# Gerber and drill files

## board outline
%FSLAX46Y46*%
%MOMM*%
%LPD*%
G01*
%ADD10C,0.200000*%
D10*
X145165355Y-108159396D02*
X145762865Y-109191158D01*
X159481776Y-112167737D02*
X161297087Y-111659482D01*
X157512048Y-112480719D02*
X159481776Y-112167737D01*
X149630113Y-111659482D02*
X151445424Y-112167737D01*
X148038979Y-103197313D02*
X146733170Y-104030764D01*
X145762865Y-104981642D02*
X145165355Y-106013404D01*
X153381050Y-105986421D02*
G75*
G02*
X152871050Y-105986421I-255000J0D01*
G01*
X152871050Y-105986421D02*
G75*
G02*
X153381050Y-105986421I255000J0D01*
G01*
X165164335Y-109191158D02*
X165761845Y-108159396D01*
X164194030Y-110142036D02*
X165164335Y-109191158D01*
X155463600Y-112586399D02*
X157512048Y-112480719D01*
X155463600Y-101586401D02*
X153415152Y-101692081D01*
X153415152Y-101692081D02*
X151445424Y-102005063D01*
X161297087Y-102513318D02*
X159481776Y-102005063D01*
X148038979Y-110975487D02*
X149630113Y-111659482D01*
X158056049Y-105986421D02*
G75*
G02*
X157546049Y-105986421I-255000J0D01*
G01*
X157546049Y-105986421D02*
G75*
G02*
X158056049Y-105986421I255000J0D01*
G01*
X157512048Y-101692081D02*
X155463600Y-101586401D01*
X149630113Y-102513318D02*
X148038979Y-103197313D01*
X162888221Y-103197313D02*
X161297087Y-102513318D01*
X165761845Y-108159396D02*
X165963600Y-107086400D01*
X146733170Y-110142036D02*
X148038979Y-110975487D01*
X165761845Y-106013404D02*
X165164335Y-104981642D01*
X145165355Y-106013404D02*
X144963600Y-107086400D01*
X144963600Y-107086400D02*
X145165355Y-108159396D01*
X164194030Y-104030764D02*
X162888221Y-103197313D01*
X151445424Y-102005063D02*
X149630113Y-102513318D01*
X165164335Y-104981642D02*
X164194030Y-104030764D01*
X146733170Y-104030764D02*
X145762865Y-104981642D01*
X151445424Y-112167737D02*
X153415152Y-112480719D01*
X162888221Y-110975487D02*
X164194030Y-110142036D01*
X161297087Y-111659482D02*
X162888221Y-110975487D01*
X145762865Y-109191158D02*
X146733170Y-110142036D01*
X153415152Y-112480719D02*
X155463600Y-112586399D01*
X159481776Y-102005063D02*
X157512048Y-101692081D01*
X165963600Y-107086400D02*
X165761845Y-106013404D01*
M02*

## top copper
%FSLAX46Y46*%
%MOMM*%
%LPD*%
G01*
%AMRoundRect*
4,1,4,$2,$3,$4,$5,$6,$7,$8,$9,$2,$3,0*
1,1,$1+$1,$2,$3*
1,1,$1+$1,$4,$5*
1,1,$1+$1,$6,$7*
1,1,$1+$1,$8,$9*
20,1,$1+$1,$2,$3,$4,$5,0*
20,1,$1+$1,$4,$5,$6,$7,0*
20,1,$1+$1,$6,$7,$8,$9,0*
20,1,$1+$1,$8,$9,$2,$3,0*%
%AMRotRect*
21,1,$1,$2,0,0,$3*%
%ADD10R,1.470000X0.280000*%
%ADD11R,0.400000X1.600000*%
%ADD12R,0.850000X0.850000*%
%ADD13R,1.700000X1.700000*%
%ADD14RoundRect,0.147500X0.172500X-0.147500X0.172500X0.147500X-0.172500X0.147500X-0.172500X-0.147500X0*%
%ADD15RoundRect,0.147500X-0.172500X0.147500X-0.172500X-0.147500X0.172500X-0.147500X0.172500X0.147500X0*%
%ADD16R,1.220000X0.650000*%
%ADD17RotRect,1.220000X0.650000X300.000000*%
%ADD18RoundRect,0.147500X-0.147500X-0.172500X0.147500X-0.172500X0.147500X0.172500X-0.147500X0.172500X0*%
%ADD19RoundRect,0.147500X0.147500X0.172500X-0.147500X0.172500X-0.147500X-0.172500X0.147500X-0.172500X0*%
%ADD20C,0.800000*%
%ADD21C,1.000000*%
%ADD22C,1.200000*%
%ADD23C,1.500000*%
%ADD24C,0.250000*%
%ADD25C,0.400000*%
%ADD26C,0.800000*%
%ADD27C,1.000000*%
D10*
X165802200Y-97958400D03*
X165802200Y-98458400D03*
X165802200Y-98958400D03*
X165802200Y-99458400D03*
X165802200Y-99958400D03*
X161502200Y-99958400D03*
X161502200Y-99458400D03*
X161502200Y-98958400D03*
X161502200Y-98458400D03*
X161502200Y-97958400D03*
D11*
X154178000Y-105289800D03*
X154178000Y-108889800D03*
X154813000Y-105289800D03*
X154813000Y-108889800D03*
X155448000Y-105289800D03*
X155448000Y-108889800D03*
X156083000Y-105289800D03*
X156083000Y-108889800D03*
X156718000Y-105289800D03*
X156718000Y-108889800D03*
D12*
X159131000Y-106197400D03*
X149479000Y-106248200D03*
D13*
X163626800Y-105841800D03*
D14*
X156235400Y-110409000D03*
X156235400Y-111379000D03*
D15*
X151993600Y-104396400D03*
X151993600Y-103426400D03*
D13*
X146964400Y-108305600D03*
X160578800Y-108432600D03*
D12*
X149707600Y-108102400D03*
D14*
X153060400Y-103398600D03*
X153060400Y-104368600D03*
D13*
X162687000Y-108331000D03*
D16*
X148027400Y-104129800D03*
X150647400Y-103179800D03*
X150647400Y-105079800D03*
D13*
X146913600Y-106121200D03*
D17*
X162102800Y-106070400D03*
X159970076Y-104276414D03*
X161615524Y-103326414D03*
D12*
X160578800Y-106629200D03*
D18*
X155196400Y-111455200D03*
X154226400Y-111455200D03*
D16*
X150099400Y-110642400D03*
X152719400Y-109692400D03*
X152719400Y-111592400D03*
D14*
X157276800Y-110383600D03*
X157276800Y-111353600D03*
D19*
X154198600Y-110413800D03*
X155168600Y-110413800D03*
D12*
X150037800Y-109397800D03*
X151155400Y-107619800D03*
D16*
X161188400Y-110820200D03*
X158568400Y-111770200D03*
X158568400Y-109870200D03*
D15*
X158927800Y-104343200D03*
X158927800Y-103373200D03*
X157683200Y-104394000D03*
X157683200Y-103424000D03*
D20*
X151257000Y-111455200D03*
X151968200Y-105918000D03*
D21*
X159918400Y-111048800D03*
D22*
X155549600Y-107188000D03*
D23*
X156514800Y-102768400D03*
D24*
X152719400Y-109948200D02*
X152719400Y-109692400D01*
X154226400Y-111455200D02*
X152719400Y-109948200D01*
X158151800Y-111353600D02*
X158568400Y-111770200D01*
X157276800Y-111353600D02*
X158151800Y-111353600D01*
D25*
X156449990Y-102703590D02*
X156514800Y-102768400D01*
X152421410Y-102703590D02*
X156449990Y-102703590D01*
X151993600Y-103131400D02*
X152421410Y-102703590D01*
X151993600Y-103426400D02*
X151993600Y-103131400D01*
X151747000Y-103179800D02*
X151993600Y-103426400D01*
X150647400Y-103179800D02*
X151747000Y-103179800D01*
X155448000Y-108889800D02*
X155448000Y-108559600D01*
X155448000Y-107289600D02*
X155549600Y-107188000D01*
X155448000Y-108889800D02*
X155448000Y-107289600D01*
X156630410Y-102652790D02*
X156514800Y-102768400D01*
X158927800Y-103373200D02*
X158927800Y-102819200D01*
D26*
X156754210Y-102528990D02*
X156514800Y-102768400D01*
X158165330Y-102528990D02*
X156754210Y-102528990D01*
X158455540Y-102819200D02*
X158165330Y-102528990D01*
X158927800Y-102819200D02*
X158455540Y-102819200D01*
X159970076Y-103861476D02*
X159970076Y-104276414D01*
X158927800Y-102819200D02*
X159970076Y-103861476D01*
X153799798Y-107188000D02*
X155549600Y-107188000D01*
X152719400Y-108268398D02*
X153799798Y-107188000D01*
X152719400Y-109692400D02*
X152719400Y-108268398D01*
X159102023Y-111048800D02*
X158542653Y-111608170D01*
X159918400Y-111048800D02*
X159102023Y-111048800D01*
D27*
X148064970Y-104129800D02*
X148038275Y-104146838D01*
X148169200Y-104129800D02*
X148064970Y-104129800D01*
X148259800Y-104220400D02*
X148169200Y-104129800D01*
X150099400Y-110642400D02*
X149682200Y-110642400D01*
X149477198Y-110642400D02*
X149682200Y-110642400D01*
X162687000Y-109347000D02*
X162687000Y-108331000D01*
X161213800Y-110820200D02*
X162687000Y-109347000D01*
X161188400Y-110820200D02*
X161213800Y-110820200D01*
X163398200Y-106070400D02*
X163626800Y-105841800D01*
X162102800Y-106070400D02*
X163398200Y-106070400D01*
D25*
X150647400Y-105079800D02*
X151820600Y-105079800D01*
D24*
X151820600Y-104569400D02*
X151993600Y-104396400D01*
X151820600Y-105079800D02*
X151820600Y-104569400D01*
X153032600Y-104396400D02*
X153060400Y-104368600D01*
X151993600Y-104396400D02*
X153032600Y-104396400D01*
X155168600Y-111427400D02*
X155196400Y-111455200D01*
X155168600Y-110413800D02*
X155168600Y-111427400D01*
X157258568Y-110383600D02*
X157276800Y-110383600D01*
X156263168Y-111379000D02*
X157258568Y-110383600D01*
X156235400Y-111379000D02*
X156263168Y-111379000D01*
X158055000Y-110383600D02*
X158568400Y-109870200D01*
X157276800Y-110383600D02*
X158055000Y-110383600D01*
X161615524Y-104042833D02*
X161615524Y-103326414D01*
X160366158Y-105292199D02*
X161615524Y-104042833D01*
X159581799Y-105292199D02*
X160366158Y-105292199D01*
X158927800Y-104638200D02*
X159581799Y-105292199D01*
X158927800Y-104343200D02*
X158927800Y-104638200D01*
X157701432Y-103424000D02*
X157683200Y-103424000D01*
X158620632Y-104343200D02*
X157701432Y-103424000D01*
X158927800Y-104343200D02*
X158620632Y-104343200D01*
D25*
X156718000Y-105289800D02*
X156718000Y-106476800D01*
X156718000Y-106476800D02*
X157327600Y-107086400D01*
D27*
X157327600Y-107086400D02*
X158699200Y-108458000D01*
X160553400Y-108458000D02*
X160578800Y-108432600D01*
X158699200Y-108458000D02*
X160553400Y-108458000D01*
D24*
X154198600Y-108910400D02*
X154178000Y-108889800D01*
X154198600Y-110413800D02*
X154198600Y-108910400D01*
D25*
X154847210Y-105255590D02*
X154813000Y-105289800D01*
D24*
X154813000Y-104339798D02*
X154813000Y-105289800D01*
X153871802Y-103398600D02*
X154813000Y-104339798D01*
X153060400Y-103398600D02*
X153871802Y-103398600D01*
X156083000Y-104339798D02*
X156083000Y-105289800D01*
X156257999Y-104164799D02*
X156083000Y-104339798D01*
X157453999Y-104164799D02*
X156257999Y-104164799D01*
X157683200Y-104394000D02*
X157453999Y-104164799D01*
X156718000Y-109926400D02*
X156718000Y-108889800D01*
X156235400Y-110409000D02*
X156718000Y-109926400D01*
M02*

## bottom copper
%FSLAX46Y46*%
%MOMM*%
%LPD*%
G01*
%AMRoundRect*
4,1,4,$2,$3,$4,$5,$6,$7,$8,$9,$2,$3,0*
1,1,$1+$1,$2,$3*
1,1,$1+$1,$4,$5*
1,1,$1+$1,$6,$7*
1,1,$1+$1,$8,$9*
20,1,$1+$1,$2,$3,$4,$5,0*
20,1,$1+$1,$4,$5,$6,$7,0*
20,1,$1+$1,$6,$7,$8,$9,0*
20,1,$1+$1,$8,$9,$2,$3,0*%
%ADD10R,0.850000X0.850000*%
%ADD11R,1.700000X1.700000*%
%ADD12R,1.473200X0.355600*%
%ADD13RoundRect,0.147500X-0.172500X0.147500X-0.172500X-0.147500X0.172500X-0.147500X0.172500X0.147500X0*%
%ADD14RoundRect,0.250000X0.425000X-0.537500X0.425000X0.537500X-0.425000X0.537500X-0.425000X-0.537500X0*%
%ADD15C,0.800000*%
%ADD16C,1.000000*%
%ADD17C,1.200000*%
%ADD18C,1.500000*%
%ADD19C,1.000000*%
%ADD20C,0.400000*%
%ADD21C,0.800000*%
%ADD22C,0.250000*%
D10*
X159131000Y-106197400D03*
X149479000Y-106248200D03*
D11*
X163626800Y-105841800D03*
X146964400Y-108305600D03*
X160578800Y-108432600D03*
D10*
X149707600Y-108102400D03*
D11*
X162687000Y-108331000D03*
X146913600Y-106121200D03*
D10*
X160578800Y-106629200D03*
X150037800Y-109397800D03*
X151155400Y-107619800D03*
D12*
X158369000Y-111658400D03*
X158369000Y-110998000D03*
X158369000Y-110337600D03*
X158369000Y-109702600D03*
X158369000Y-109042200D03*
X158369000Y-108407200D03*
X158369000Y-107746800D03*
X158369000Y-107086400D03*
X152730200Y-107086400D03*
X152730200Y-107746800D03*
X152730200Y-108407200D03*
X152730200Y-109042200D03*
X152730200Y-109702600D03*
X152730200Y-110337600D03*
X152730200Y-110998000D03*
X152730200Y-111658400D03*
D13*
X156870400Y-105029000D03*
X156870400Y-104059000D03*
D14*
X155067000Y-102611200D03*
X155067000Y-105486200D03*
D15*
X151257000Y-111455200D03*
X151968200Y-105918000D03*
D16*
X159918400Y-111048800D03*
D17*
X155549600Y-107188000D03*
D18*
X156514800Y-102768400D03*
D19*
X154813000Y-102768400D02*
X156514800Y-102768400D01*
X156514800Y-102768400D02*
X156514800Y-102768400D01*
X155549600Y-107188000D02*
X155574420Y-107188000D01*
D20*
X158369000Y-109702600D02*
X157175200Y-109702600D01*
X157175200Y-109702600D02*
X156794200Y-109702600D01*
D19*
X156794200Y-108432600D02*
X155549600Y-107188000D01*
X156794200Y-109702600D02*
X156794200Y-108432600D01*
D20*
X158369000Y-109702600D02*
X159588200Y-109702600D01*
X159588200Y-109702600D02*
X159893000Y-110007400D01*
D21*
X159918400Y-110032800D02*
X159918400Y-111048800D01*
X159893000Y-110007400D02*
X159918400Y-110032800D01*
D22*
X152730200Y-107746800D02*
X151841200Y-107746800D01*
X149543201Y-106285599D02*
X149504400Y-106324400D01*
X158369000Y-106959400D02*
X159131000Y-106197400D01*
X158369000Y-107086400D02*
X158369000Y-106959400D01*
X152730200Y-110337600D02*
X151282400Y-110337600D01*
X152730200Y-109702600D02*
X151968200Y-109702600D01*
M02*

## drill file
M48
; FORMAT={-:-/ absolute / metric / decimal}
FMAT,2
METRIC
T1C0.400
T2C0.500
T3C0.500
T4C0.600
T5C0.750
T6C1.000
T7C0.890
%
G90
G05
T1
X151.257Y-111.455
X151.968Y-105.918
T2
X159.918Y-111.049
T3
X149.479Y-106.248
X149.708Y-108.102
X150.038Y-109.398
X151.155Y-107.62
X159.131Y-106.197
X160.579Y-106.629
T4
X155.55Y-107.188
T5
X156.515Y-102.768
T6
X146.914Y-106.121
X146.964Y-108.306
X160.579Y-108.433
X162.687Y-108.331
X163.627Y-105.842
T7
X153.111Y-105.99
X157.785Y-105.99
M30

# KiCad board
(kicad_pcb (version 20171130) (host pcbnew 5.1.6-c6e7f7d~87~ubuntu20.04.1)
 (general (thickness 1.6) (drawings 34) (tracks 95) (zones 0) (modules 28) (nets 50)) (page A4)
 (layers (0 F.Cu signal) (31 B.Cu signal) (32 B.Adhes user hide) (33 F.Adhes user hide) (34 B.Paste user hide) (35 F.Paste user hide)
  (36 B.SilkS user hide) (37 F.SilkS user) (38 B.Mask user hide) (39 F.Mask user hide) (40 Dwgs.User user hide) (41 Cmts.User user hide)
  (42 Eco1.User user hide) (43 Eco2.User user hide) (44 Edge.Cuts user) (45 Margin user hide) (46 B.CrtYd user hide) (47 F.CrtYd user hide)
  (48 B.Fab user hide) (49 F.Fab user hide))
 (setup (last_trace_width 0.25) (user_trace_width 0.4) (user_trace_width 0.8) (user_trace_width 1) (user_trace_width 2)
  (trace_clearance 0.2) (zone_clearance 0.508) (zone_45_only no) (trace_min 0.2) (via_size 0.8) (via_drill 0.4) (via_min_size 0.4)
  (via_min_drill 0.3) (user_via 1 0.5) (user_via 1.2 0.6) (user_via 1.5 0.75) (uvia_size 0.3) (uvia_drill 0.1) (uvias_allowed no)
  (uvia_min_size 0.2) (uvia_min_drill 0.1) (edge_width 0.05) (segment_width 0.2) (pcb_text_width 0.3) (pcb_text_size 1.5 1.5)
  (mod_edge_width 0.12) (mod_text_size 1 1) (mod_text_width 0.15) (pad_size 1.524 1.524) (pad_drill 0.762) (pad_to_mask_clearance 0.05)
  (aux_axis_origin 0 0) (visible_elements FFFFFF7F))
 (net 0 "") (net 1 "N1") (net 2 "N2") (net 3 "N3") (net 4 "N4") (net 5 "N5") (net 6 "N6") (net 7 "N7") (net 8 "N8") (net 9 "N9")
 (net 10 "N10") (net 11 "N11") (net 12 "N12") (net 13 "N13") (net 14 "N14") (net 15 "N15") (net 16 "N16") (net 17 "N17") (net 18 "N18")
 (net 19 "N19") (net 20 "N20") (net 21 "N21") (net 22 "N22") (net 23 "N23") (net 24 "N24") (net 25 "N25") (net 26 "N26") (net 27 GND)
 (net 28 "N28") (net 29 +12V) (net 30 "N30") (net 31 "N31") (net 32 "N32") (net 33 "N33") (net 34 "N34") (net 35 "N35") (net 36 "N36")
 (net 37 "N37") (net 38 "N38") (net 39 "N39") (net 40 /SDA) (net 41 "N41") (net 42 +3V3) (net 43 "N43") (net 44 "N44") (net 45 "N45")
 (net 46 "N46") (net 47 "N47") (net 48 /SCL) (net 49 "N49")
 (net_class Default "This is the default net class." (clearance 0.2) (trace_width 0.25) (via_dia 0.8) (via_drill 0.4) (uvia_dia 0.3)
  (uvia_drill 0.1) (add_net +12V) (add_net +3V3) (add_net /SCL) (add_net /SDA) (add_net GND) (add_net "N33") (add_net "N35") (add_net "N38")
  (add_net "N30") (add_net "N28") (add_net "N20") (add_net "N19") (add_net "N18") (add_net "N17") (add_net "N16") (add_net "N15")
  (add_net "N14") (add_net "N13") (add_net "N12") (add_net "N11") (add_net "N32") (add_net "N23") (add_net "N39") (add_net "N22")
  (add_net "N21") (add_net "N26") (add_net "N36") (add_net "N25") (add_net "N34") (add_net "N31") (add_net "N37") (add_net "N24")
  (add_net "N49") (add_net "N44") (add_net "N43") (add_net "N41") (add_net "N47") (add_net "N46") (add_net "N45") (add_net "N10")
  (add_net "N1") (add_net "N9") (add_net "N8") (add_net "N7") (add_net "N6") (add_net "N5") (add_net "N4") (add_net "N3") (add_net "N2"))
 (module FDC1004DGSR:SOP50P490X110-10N (layer F.Cu) (at 163.6522 98.9584)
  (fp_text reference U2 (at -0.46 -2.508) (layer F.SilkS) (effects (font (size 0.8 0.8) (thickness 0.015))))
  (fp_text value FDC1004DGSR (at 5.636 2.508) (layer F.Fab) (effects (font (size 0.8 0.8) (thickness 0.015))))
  (pad 10 smd rect (at 2.15 -1) (size 1.47 0.28) (layers F.Cu F.Paste F.Mask) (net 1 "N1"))
  (pad 9 smd rect (at 2.15 -0.5) (size 1.47 0.28) (layers F.Cu F.Paste F.Mask) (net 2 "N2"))
  (pad 8 smd rect (at 2.15 0) (size 1.47 0.28) (layers F.Cu F.Paste F.Mask) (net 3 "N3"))
  (pad 7 smd rect (at 2.15 0.5) (size 1.47 0.28) (layers F.Cu F.Paste F.Mask) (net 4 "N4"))
  (pad 6 smd rect (at 2.15 1) (size 1.47 0.28) (layers F.Cu F.Paste F.Mask) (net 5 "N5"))
  (pad 5 smd rect (at -2.15 1) (size 1.47 0.28) (layers F.Cu F.Paste F.Mask) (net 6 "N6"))
  (pad 4 smd rect (at -2.15 0.5) (size 1.47 0.28) (layers F.Cu F.Paste F.Mask) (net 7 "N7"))
  (pad 3 smd rect (at -2.15 0) (size 1.47 0.28) (layers F.Cu F.Paste F.Mask) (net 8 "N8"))
  (pad 2 smd rect (at -2.15 -0.5) (size 1.47 0.28) (layers F.Cu F.Paste F.Mask) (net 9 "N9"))
  (pad 1 smd rect (at -2.15 -1) (size 1.47 0.28) (layers F.Cu F.Paste F.Mask) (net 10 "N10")))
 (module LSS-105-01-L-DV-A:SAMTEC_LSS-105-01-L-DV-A (layer F.Cu) (at 156.718 108.8898)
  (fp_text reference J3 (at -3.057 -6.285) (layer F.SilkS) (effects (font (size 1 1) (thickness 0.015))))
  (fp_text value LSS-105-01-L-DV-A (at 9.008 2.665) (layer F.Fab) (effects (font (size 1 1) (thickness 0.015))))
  (pad 10 smd rect (at -2.54 -3.6) (size 0.4 1.6) (layers F.Cu F.Paste F.Mask) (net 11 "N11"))
  (pad 09 smd rect (at -2.54 0) (size 0.4 1.6) (layers F.Cu F.Paste F.Mask) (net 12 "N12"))
  (pad 08 smd rect (at -1.905 -3.6) (size 0.4 1.6) (layers F.Cu F.Paste F.Mask) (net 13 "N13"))
  (pad 07 smd rect (at -1.905 0) (size 0.4 1.6) (layers F.Cu F.Paste F.Mask) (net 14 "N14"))
  (pad 06 smd rect (at -1.27 -3.6) (size 0.4 1.6) (layers F.Cu F.Paste F.Mask) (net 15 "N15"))
  (pad 05 smd rect (at -1.27 0) (size 0.4 1.6) (layers F.Cu F.Paste F.Mask) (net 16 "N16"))
  (pad 04 smd rect (at -0.635 -3.6) (size 0.4 1.6) (layers F.Cu F.Paste F.Mask) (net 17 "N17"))
  (pad 03 smd rect (at -0.635 0) (size 0.4 1.6) (layers F.Cu F.Paste F.Mask) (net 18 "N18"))
  (pad 02 smd rect (at 0 -3.6) (size 0.4 1.6) (layers F.Cu F.Paste F.Mask) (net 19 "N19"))
  (pad 01 smd rect (at 0 0) (size 0.4 1.6) (layers F.Cu F.Paste F.Mask) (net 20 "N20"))
  (pad None np_thru_hole circle (at 1.067 -2.9) (size 0.89 0.89) (drill 0.89) (layers *.Cu *.Mask))
  (pad None np_thru_hole circle (at -3.607 -2.9) (size 0.89 0.89) (drill 0.89) (layers *.Cu *.Mask)))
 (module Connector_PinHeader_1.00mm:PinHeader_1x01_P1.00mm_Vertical (layer F.Cu) (at 159.131 106.1974)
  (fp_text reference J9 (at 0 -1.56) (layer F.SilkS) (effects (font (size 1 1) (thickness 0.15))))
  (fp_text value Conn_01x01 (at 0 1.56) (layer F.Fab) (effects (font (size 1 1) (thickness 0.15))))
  (pad 1 thru_hole rect (at 0 0) (size 0.85 0.85) (drill 0.5) (layers *.Cu *.Mask) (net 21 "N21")))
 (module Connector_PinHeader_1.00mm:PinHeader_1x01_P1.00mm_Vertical (layer F.Cu) (at 149.479 106.2482)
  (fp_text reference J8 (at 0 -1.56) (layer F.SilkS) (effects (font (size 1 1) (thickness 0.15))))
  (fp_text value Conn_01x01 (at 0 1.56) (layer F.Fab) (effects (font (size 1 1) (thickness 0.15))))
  (pad 1 thru_hole rect (at 0 0) (size 0.85 0.85) (drill 0.5) (layers *.Cu *.Mask) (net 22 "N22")))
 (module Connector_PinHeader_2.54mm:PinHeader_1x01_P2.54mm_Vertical (layer F.Cu) (at 163.6268 105.8418)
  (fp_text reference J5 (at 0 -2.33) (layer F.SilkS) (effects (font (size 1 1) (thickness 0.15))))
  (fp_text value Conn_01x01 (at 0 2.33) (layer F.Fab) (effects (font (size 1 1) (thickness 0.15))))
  (pad 1 thru_hole rect (at 0 0) (size 1.7 1.7) (drill 1) (layers *.Cu *.Mask) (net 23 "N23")))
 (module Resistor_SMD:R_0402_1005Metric (layer F.Cu) (at 156.2354 110.894 90)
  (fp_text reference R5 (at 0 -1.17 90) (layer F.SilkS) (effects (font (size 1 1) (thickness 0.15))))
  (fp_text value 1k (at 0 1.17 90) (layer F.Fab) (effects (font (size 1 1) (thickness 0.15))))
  (pad 2 smd roundrect (at 0.485 0 90) (size 0.59 0.64) (layers F.Cu F.Paste F.Mask) (roundrect_rratio 0.25) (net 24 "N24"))
  (pad 1 smd roundrect (at -0.485 0 90) (size 0.59 0.64) (layers F.Cu F.Paste F.Mask) (roundrect_rratio 0.25) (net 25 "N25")))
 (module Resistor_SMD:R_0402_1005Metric (layer F.Cu) (at 151.9936 103.9114 270)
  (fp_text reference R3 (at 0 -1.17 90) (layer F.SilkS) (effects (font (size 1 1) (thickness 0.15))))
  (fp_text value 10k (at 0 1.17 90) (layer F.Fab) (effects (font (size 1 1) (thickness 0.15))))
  (pad 2 smd roundrect (at 0.485 0 270) (size 0.59 0.64) (layers F.Cu F.Paste F.Mask) (roundrect_rratio 0.25) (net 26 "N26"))
  (pad 1 smd roundrect (at -0.485 0 270) (size 0.59 0.64) (layers F.Cu F.Paste F.Mask) (roundrect_rratio 0.25) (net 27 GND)))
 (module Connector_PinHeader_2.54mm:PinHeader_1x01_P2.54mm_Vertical (layer F.Cu) (at 146.9644 108.3056)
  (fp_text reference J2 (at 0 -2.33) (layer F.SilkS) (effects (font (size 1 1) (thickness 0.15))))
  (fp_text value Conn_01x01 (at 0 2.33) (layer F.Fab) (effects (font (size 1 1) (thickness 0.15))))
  (pad 1 thru_hole rect (at 0 0) (size 1.7 1.7) (drill 1) (layers *.Cu *.Mask) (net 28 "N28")))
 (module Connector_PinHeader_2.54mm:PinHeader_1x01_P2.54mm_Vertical (layer F.Cu) (at 160.5788 108.4326)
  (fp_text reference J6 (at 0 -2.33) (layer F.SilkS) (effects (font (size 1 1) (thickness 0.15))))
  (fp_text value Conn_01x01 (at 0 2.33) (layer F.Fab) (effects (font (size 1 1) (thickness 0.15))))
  (pad 1 thru_hole rect (at 0 0) (size 1.7 1.7) (drill 1) (layers *.Cu *.Mask) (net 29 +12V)))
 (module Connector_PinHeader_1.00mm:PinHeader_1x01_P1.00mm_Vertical (layer F.Cu) (at 149.7076 108.1024)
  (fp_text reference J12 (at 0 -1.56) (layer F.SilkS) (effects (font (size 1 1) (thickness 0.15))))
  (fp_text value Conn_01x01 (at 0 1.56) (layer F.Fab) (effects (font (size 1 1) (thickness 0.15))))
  (pad 1 thru_hole rect (at 0 0) (size 0.85 0.85) (drill 0.5) (layers *.Cu *.Mask) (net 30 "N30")))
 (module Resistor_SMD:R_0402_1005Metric (layer F.Cu) (at 153.0604 103.8836 90)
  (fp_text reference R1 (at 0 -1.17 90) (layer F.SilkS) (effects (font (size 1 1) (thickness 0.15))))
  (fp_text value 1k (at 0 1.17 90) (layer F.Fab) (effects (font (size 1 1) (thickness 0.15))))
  (pad 2 smd roundrect (at 0.485 0 90) (size 0.59 0.64) (layers F.Cu F.Paste F.Mask) (roundrect_rratio 0.25) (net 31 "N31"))
  (pad 1 smd roundrect (at -0.485 0 90) (size 0.59 0.64) (layers F.Cu F.Paste F.Mask) (roundrect_rratio 0.25) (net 26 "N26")))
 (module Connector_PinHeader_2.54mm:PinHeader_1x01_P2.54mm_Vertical (layer F.Cu) (at 162.687 108.331)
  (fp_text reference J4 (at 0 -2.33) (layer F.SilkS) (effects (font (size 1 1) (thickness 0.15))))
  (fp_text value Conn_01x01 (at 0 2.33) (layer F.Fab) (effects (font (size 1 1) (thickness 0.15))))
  (pad 1 thru_hole rect (at 0 0) (size 1.7 1.7) (drill 1) (layers *.Cu *.Mask) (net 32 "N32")))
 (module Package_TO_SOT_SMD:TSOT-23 (layer F.Cu) (at 149.3374 104.1298 180)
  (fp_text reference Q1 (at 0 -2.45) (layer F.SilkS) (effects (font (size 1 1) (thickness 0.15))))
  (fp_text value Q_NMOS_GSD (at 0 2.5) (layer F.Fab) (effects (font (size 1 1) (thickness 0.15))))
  (pad 3 smd rect (at 1.31 0 180) (size 1.22 0.65) (layers F.Cu F.Paste F.Mask) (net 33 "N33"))
  (pad 2 smd rect (at -1.31 0.95 180) (size 1.22 0.65) (layers F.Cu F.Paste F.Mask) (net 27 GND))
  (pad 1 smd rect (at -1.31 -0.95 180) (size 1.22 0.65) (layers F.Cu F.Paste F.Mask) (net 26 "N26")))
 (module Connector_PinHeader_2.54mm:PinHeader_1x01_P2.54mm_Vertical (layer F.Cu) (at 146.9136 106.1212)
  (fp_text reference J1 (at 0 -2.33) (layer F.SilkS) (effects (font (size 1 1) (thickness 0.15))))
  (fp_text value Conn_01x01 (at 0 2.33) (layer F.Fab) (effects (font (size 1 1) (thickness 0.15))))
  (pad 1 thru_hole rect (at 0 0) (size 1.7 1.7) (drill 1) (layers *.Cu *.Mask) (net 33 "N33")))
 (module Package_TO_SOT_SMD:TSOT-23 (layer F.Cu) (at 161.4478 104.935907 300)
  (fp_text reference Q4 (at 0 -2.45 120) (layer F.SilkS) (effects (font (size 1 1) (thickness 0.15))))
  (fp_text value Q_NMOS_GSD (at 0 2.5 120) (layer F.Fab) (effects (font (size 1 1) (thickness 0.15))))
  (pad 3 smd rect (at 1.31 0 300) (size 1.22 0.65) (layers F.Cu F.Paste F.Mask) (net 23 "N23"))
  (pad 2 smd rect (at -1.31 0.95 300) (size 1.22 0.65) (layers F.Cu F.Paste F.Mask) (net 27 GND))
  (pad 1 smd rect (at -1.31 -0.95 300) (size 1.22 0.65) (layers F.Cu F.Paste F.Mask) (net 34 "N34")))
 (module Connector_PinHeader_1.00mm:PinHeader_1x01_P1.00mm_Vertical (layer F.Cu) (at 160.5788 106.6292)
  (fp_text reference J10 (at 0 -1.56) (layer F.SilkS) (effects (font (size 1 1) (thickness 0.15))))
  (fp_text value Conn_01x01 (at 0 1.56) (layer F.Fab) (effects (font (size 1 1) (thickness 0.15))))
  (pad 1 thru_hole rect (at 0 0) (size 0.85 0.85) (drill 0.5) (layers *.Cu *.Mask) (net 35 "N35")))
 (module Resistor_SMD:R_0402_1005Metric (layer F.Cu) (at 154.7114 111.4552)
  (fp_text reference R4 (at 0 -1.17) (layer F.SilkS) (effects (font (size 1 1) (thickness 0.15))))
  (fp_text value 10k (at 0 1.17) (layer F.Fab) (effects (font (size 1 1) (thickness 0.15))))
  (pad 2 smd roundrect (at 0.485 0) (size 0.59 0.64) (layers F.Cu F.Paste F.Mask) (roundrect_rratio 0.25) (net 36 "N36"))
  (pad 1 smd roundrect (at -0.485 0) (size 0.59 0.64) (layers F.Cu F.Paste F.Mask) (roundrect_rratio 0.25) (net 27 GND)))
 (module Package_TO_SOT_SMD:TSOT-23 (layer F.Cu) (at 151.4094 110.6424 180)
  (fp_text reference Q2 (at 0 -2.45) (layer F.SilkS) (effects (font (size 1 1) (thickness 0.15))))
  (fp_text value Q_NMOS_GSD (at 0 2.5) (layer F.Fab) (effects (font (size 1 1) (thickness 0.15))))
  (pad 3 smd rect (at 1.31 0 180) (size 1.22 0.65) (layers F.Cu F.Paste F.Mask) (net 28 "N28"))
  (pad 2 smd rect (at -1.31 0.95 180) (size 1.22 0.65) (layers F.Cu F.Paste F.Mask) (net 27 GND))
  (pad 1 smd rect (at -1.31 -0.95 180) (size 1.22 0.65) (layers F.Cu F.Paste F.Mask) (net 36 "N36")))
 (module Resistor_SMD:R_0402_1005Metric (layer F.Cu) (at 157.2768 110.8686 90)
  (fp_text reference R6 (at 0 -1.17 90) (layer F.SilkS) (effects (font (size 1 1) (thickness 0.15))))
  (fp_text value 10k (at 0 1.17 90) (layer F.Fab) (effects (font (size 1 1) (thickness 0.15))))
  (pad 2 smd roundrect (at 0.485 0 90) (size 0.59 0.64) (layers F.Cu F.Paste F.Mask) (roundrect_rratio 0.25) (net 25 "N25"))
  (pad 1 smd roundrect (at -0.485 0 90) (size 0.59 0.64) (layers F.Cu F.Paste F.Mask) (roundrect_rratio 0.25) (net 27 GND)))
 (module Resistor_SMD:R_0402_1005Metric (layer F.Cu) (at 154.6836 110.4138 180)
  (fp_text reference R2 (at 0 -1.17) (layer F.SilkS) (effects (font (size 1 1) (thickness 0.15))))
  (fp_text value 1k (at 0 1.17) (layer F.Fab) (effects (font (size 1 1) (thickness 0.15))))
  (pad 2 smd roundrect (at 0.485 0 180) (size 0.59 0.64) (layers F.Cu F.Paste F.Mask) (roundrect_rratio 0.25) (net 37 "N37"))
  (pad 1 smd roundrect (at -0.485 0 180) (size 0.59 0.64) (layers F.Cu F.Paste F.Mask) (roundrect_rratio 0.25) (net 36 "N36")))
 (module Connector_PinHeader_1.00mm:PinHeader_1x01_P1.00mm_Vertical (layer F.Cu) (at 150.0378 109.3978)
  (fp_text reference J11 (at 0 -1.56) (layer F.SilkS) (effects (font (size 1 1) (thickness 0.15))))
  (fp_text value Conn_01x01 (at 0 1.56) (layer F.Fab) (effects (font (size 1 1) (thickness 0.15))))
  (pad 1 thru_hole rect (at 0 0) (size 0.85 0.85) (drill 0.5) (layers *.Cu *.Mask) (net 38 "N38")))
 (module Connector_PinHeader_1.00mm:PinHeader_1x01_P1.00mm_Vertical (layer F.Cu) (at 151.1554 107.6198)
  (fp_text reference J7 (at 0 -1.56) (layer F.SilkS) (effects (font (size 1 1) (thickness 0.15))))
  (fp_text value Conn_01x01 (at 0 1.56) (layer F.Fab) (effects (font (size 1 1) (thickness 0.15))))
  (pad 1 thru_hole rect (at 0 0) (size 0.85 0.85) (drill 0.5) (layers *.Cu *.Mask) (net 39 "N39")))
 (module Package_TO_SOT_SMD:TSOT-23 (layer F.Cu) (at 159.8784 110.8202)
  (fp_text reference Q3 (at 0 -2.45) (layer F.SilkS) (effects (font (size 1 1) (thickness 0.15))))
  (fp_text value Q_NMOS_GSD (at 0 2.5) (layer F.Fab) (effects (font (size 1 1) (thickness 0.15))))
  (pad 3 smd rect (at 1.31 0) (size 1.22 0.65) (layers F.Cu F.Paste F.Mask) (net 32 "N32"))
  (pad 2 smd rect (at -1.31 0.95) (size 1.22 0.65) (layers F.Cu F.Paste F.Mask) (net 27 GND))
  (pad 1 smd rect (at -1.31 -0.95) (size 1.22 0.65) (layers F.Cu F.Paste F.Mask) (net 25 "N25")))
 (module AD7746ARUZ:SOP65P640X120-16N (layer B.Cu) (at 155.5496 109.3724)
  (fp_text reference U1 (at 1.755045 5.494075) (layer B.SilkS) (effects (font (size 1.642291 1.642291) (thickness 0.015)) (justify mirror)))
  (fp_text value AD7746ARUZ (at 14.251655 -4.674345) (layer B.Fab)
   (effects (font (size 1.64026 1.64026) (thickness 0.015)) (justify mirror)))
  (pad 16 smd rect (at 2.8194 2.286) (size 1.4732 0.3556) (layers B.Cu B.Paste B.Mask) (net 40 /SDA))
  (pad 15 smd rect (at 2.8194 1.6256) (size 1.4732 0.3556) (layers B.Cu B.Paste B.Mask) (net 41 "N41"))
  (pad 14 smd rect (at 2.8194 0.9652) (size 1.4732 0.3556) (layers B.Cu B.Paste B.Mask) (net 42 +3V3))
  (pad 13 smd rect (at 2.8194 0.3302) (size 1.4732 0.3556) (layers B.Cu B.Paste B.Mask) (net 27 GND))
  (pad 12 smd rect (at 2.8194 -0.3302) (size 1.4732 0.3556) (layers B.Cu B.Paste B.Mask) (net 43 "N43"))
  (pad 11 smd rect (at 2.8194 -0.9652) (size 1.4732 0.3556) (layers B.Cu B.Paste B.Mask) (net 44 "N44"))
  (pad 10 smd rect (at 2.8194 -1.6256) (size 1.4732 0.3556) (layers B.Cu B.Paste B.Mask) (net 35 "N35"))
  (pad 9 smd rect (at 2.8194 -2.286) (size 1.4732 0.3556) (layers B.Cu B.Paste B.Mask) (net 21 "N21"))
  (pad 8 smd rect (at -2.8194 -2.286) (size 1.4732 0.3556) (layers B.Cu B.Paste B.Mask) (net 22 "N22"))
  (pad 7 smd rect (at -2.8194 -1.6256) (size 1.4732 0.3556) (layers B.Cu B.Paste B.Mask) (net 39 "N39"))
  (pad 6 smd rect (at -2.8194 -0.9652) (size 1.4732 0.3556) (layers B.Cu B.Paste B.Mask) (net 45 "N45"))
  (pad 5 smd rect (at -2.8194 -0.3302) (size 1.4732 0.3556) (layers B.Cu B.Paste B.Mask) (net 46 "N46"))
  (pad 4 smd rect (at -2.8194 0.3302) (size 1.4732 0.3556) (layers B.Cu B.Paste B.Mask) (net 30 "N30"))
  (pad 3 smd rect (at -2.8194 0.9652) (size 1.4732 0.3556) (layers B.Cu B.Paste B.Mask) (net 38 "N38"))
  (pad 2 smd rect (at -2.8194 1.6256) (size 1.4732 0.3556) (layers B.Cu B.Paste B.Mask) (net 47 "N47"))
  (pad 1 smd rect (at -2.8194 2.286) (size 1.4732 0.3556) (layers B.Cu B.Paste B.Mask) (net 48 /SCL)))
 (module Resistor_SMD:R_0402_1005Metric (layer F.Cu) (at 158.9278 103.8582 270)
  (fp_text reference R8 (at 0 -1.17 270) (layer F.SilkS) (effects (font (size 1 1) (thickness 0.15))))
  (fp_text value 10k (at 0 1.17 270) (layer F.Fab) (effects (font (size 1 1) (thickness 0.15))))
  (pad 2 smd roundrect (at 0.485 0 270) (size 0.59 0.64) (layers F.Cu F.Paste F.Mask) (roundrect_rratio 0.25) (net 34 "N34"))
  (pad 1 smd roundrect (at -0.485 0 270) (size 0.59 0.64) (layers F.Cu F.Paste F.Mask) (roundrect_rratio 0.25) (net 27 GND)))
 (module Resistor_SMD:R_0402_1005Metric (layer F.Cu) (at 157.6832 103.909 270)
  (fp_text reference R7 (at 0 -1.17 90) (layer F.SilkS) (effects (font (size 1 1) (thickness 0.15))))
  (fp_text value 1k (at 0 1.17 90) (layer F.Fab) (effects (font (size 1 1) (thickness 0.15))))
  (pad 2 smd roundrect (at 0.485 0 270) (size 0.59 0.64) (layers F.Cu F.Paste F.Mask) (roundrect_rratio 0.25) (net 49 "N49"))
  (pad 1 smd roundrect (at -0.485 0 270) (size 0.59 0.64) (layers F.Cu F.Paste F.Mask) (roundrect_rratio 0.25) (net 34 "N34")))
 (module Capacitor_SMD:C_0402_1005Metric (layer B.Cu) (at 156.8704 104.544 270)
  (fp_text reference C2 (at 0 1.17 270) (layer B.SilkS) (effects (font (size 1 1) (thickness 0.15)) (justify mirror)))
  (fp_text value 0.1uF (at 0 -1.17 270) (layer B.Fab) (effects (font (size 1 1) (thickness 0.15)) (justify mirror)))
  (pad 2 smd roundrect (at 0.485 0 270) (size 0.59 0.64) (layers B.Cu B.Paste B.Mask) (roundrect_rratio 0.25) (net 27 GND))
  (pad 1 smd roundrect (at -0.485 0 270) (size 0.59 0.64) (layers B.Cu B.Paste B.Mask) (roundrect_rratio 0.25) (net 42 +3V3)))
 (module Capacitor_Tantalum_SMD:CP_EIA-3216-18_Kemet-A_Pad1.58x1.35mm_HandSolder (layer B.Cu) (at 155.067 104.0487 90)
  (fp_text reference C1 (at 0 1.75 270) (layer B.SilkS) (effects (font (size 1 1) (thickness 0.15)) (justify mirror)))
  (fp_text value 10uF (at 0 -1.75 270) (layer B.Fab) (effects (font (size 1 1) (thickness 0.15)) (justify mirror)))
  (pad 2 smd roundrect (at 1.4375 0 90) (size 1.575 1.35) (layers B.Cu B.Paste B.Mask) (roundrect_rratio 0.185185) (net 27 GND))
  (pad 1 smd roundrect (at -1.4375 0 90) (size 1.575 1.35) (layers B.Cu B.Paste B.Mask) (roundrect_rratio 0.185185) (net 42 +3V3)))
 (gr_line (start 145.165355 108.159396) (end 145.762865 109.191158) (layer Edge.Cuts) (width 0.2))
 (gr_line (start 159.481776 112.167737) (end 161.297087 111.659482) (layer Edge.Cuts) (width 0.2))
 (gr_line (start 157.512048 112.480719) (end 159.481776 112.167737) (layer Edge.Cuts) (width 0.2))
 (gr_line (start 149.630113 111.659482) (end 151.445424 112.167737) (layer Edge.Cuts) (width 0.2))
 (gr_line (start 148.038979 103.197313) (end 146.73317 104.030764) (layer Edge.Cuts) (width 0.2))
 (gr_line (start 145.762865 104.981642) (end 145.165355 106.013404) (layer Edge.Cuts) (width 0.2))
 (gr_circle (center 153.12605 105.986421) (end 153.38105 105.986421) (layer Edge.Cuts) (width 0.2))
 (gr_line (start 165.164335 109.191158) (end 165.761845 108.159396) (layer Edge.Cuts) (width 0.2))
 (gr_line (start 164.19403 110.142036) (end 165.164335 109.191158) (layer Edge.Cuts) (width 0.2))
 (gr_line (start 155.4636 112.586399) (end 157.512048 112.480719) (layer Edge.Cuts) (width 0.2))
 (gr_line (start 155.4636 101.586401) (end 153.415152 101.692081) (layer Edge.Cuts) (width 0.2))
 (gr_line (start 153.415152 101.692081) (end 151.445424 102.005063) (layer Edge.Cuts) (width 0.2))
 (gr_line (start 161.297087 102.513318) (end 159.481776 102.005063) (layer Edge.Cuts) (width 0.2))
 (gr_line (start 148.038979 110.975487) (end 149.630113 111.659482) (layer Edge.Cuts) (width 0.2))
 (gr_circle (center 157.801049 105.986421) (end 158.056049 105.986421) (layer Edge.Cuts) (width 0.2))
 (gr_line (start 157.512048 101.692081) (end 155.4636 101.586401) (layer Edge.Cuts) (width 0.2))
 (gr_line (start 149.630113 102.513318) (end 148.038979 103.197313) (layer Edge.Cuts) (width 0.2))
 (gr_line (start 162.888221 103.197313) (end 161.297087 102.513318) (layer Edge.Cuts) (width 0.2))
 (gr_line (start 165.761845 108.159396) (end 165.9636 107.0864) (layer Edge.Cuts) (width 0.2))
 (gr_line (start 146.73317 110.142036) (end 148.038979 110.975487) (layer Edge.Cuts) (width 0.2))
 (gr_line (start 165.761845 106.013404) (end 165.164335 104.981642) (layer Edge.Cuts) (width 0.2))
 (gr_line (start 145.165355 106.013404) (end 144.9636 107.0864) (layer Edge.Cuts) (width 0.2))
 (gr_line (start 144.9636 107.0864) (end 145.165355 108.159396) (layer Edge.Cuts) (width 0.2))
 (gr_line (start 164.19403 104.030764) (end 162.888221 103.197313) (layer Edge.Cuts) (width 0.2))
 (gr_line (start 151.445424 102.005063) (end 149.630113 102.513318) (layer Edge.Cuts) (width 0.2))
 (gr_line (start 165.164335 104.981642) (end 164.19403 104.030764) (layer Edge.Cuts) (width 0.2))
 (gr_line (start 146.73317 104.030764) (end 145.762865 104.981642) (layer Edge.Cuts) (width 0.2))
 (gr_line (start 151.445424 112.167737) (end 153.415152 112.480719) (layer Edge.Cuts) (width 0.2))
 (gr_line (start 162.888221 110.975487) (end 164.19403 110.142036) (layer Edge.Cuts) (width 0.2))
 (gr_line (start 161.297087 111.659482) (end 162.888221 110.975487) (layer Edge.Cuts) (width 0.2))
 (gr_line (start 145.762865 109.191158) (end 146.73317 110.142036) (layer Edge.Cuts) (width 0.2))
 (gr_line (start 153.415152 112.480719) (end 155.4636 112.586399) (layer Edge.Cuts) (width 0.2))
 (gr_line (start 159.481776 102.005063) (end 157.512048 101.692081) (layer Edge.Cuts) (width 0.2))
 (gr_line (start 165.9636 107.0864) (end 165.761845 106.013404) (layer Edge.Cuts) (width 0.2))
 (via (at 151.257 111.4552) (size 0.8) (drill 0.4) (layers F.Cu B.Cu) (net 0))
 (via (at 151.9682 105.918) (size 0.8) (drill 0.4) (layers F.Cu B.Cu) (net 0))
 (via (at 159.9184 111.0488) (size 1) (drill 0.5) (layers F.Cu B.Cu) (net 27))
 (via (at 155.5496 107.188) (size 1.2) (drill 0.6) (layers F.Cu B.Cu) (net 27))
 (segment (start 152.7194 109.9482) (end 152.7194 109.6924) (width 0.25) (layer F.Cu) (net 27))
 (segment (start 154.2264 111.4552) (end 152.7194 109.9482) (width 0.25) (layer F.Cu) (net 27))
 (segment (start 158.1518 111.3536) (end 158.5684 111.7702) (width 0.25) (layer F.Cu) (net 27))
 (segment (start 157.2768 111.3536) (end 158.1518 111.3536) (width 0.25) (layer F.Cu) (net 27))
 (segment (start 154.813 102.7684) (end 156.5148 102.7684) (width 1) (layer B.Cu) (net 27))
 (segment (start 156.5148 102.7684) (end 156.5148 102.7684) (width 1) (layer B.Cu) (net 27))
 (via (at 156.5148 102.7684) (size 1.5) (drill 0.75) (layers F.Cu B.Cu) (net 27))
 (segment (start 156.44999 102.70359) (end 156.5148 102.7684) (width 0.4) (layer F.Cu) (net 27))
 (segment (start 152.42141 102.70359) (end 156.44999 102.70359) (width 0.4) (layer F.Cu) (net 27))
 (segment (start 151.9936 103.1314) (end 152.42141 102.70359) (width 0.4) (layer F.Cu) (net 27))
 (segment (start 151.9936 103.4264) (end 151.9936 103.1314) (width 0.4) (layer F.Cu) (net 27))
 (segment (start 151.747 103.1798) (end 151.9936 103.4264) (width 0.4) (layer F.Cu) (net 27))
 (segment (start 150.6474 103.1798) (end 151.747 103.1798) (width 0.4) (layer F.Cu) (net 27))
 (segment (start 155.448 108.8898) (end 155.448 108.5596) (width 0.4) (layer F.Cu) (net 27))
 (segment (start 155.448 107.2896) (end 155.5496 107.188) (width 0.4) (layer F.Cu) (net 27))
 (segment (start 155.448 108.8898) (end 155.448 107.2896) (width 0.4) (layer F.Cu) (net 27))
 (segment (start 155.5496 107.188) (end 155.57442 107.188) (width 1) (layer B.Cu) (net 27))
 (segment (start 156.63041 102.65279) (end 156.5148 102.7684) (width 0.4) (layer F.Cu) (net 27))
 (segment (start 158.9278 103.3732) (end 158.9278 102.8192) (width 0.4) (layer F.Cu) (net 27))
 (segment (start 156.75421 102.52899) (end 156.5148 102.7684) (width 0.8) (layer F.Cu) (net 27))
 (segment (start 158.16533 102.52899) (end 156.75421 102.52899) (width 0.8) (layer F.Cu) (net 27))
 (segment (start 158.45554 102.8192) (end 158.16533 102.52899) (width 0.8) (layer F.Cu) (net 27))
 (segment (start 158.9278 102.8192) (end 158.45554 102.8192) (width 0.8) (layer F.Cu) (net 27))
 (segment (start 159.970076 103.861476) (end 159.970076 104.276414) (width 0.8) (layer F.Cu) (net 27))
 (segment (start 158.9278 102.8192) (end 159.970076 103.861476) (width 0.8) (layer F.Cu) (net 27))
 (segment (start 153.799798 107.188) (end 155.5496 107.188) (width 0.8) (layer F.Cu) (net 27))
 (segment (start 152.7194 108.268398) (end 153.799798 107.188) (width 0.8) (layer F.Cu) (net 27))
 (segment (start 152.7194 109.6924) (end 152.7194 108.268398) (width 0.8) (layer F.Cu) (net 27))
 (segment (start 158.369 109.7026) (end 157.1752 109.7026) (width 0.4) (layer B.Cu) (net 27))
 (segment (start 157.1752 109.7026) (end 156.7942 109.7026) (width 0.4) (layer B.Cu) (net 27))
 (segment (start 156.7942 108.4326) (end 155.5496 107.188) (width 1) (layer B.Cu) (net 27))
 (segment (start 156.7942 109.7026) (end 156.7942 108.4326) (width 1) (layer B.Cu) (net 27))
 (segment (start 158.369 109.7026) (end 159.5882 109.7026) (width 0.4) (layer B.Cu) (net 27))
 (segment (start 159.5882 109.7026) (end 159.893 110.0074) (width 0.4) (layer B.Cu) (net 27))
 (segment (start 159.9184 110.0328) (end 159.9184 111.0488) (width 0.8) (layer B.Cu) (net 27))
 (segment (start 159.893 110.0074) (end 159.9184 110.0328) (width 0.8) (layer B.Cu) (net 27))
 (segment (start 159.102023 111.0488) (end 158.542653 111.60817) (width 0.8) (layer F.Cu) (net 27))
 (segment (start 159.9184 111.0488) (end 159.102023 111.0488) (width 0.8) (layer F.Cu) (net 27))
 (segment (start 148.06497 104.1298) (end 148.038275 104.146838) (width 1) (layer F.Cu) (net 33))
 (segment (start 148.1692 104.1298) (end 148.06497 104.1298) (width 1) (layer F.Cu) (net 33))
 (segment (start 148.2598 104.2204) (end 148.1692 104.1298) (width 1) (layer F.Cu) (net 33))
 (segment (start 150.0994 110.6424) (end 149.6822 110.6424) (width 1) (layer F.Cu) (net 28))
 (segment (start 149.477198 110.6424) (end 149.6822 110.6424) (width 1) (layer F.Cu) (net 28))
 (segment (start 162.687 109.347) (end 162.687 108.331) (width 1) (layer F.Cu) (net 32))
 (segment (start 161.2138 110.8202) (end 162.687 109.347) (width 1) (layer F.Cu) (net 32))
 (segment (start 161.1884 110.8202) (end 161.2138 110.8202) (width 1) (layer F.Cu) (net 32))
 (segment (start 163.3982 106.0704) (end 163.6268 105.8418) (width 1) (layer F.Cu) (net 23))
 (segment (start 162.1028 106.0704) (end 163.3982 106.0704) (width 1) (layer F.Cu) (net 23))
 (segment (start 150.6474 105.0798) (end 151.8206 105.0798) (width 0.4) (layer F.Cu) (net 26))
 (segment (start 151.8206 104.5694) (end 151.9936 104.3964) (width 0.25) (layer F.Cu) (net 26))
 (segment (start 151.8206 105.0798) (end 151.8206 104.5694) (width 0.25) (layer F.Cu) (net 26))
 (segment (start 153.0326 104.3964) (end 153.0604 104.3686) (width 0.25) (layer F.Cu) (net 26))
 (segment (start 151.9936 104.3964) (end 153.0326 104.3964) (width 0.25) (layer F.Cu) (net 26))
 (segment (start 155.1686 111.4274) (end 155.1964 111.4552) (width 0.25) (layer F.Cu) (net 36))
 (segment (start 155.1686 110.4138) (end 155.1686 111.4274) (width 0.25) (layer F.Cu) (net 36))
 (segment (start 157.258568 110.3836) (end 157.2768 110.3836) (width 0.25) (layer F.Cu) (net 25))
 (segment (start 156.263168 111.379) (end 157.258568 110.3836) (width 0.25) (layer F.Cu) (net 25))
 (segment (start 156.2354 111.379) (end 156.263168 111.379) (width 0.25) (layer F.Cu) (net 25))
 (segment (start 158.055 110.3836) (end 158.5684 109.8702) (width 0.25) (layer F.Cu) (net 25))
 (segment (start 157.2768 110.3836) (end 158.055 110.3836) (width 0.25) (layer F.Cu) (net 25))
 (segment (start 161.615524 104.042833) (end 161.615524 103.326414) (width 0.25) (layer F.Cu) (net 34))
 (segment (start 160.366158 105.292199) (end 161.615524 104.042833) (width 0.25) (layer F.Cu) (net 34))
 (segment (start 159.581799 105.292199) (end 160.366158 105.292199) (width 0.25) (layer F.Cu) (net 34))
 (segment (start 158.9278 104.6382) (end 159.581799 105.292199) (width 0.25) (layer F.Cu) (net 34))
 (segment (start 158.9278 104.3432) (end 158.9278 104.6382) (width 0.25) (layer F.Cu) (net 34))
 (segment (start 157.701432 103.424) (end 157.6832 103.424) (width 0.25) (layer F.Cu) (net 34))
 (segment (start 158.620632 104.3432) (end 157.701432 103.424) (width 0.25) (layer F.Cu) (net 34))
 (segment (start 158.9278 104.3432) (end 158.620632 104.3432) (width 0.25) (layer F.Cu) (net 34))
 (segment (start 156.718 105.2898) (end 156.718 106.4768) (width 0.4) (layer F.Cu) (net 29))
 (segment (start 156.718 106.4768) (end 157.3276 107.0864) (width 0.4) (layer F.Cu) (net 29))
 (segment (start 157.3276 107.0864) (end 158.6992 108.458) (width 1) (layer F.Cu) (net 29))
 (segment (start 160.5534 108.458) (end 160.5788 108.4326) (width 1) (layer F.Cu) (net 29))
 (segment (start 158.6992 108.458) (end 160.5534 108.458) (width 1) (layer F.Cu) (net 29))
 (segment (start 152.7302 107.7468) (end 151.8412 107.7468) (width 0.25) (layer B.Cu) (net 39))
 (segment (start 149.543201 106.285599) (end 149.5044 106.3244) (width 0.25) (layer B.Cu) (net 22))
 (segment (start 158.369 106.9594) (end 159.131 106.1974) (width 0.25) (layer B.Cu) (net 21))
 (segment (start 158.369 107.0864) (end 158.369 106.9594) (width 0.25) (layer B.Cu) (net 21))
 (segment (start 152.7302 110.3376) (end 151.2824 110.3376) (width 0.25) (layer B.Cu) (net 38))
 (segment (start 152.7302 109.7026) (end 151.9682 109.7026) (width 0.25) (layer B.Cu) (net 30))
 (segment (start 154.1986 108.9104) (end 154.178 108.8898) (width 0.25) (layer F.Cu) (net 12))
 (segment (start 154.1986 110.4138) (end 154.1986 108.9104) (width 0.25) (layer F.Cu) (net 12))
 (segment (start 154.84721 105.25559) (end 154.813 105.2898) (width 0.4) (layer F.Cu) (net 13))
 (segment (start 154.813 104.339798) (end 154.813 105.2898) (width 0.25) (layer F.Cu) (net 13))
 (segment (start 153.871802 103.3986) (end 154.813 104.339798) (width 0.25) (layer F.Cu) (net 13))
 (segment (start 153.0604 103.3986) (end 153.871802 103.3986) (width 0.25) (layer F.Cu) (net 13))
 (segment (start 156.083 104.339798) (end 156.083 105.2898) (width 0.25) (layer F.Cu) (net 17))
 (segment (start 156.257999 104.164799) (end 156.083 104.339798) (width 0.25) (layer F.Cu) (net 17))
 (segment (start 157.453999 104.164799) (end 156.257999 104.164799) (width 0.25) (layer F.Cu) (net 17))
 (segment (start 157.6832 104.394) (end 157.453999 104.164799) (width 0.25) (layer F.Cu) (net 17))
 (segment (start 156.718 109.9264) (end 156.718 108.8898) (width 0.25) (layer F.Cu) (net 20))
 (segment (start 156.2354 110.409) (end 156.718 109.9264) (width 0.25) (layer F.Cu) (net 20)))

